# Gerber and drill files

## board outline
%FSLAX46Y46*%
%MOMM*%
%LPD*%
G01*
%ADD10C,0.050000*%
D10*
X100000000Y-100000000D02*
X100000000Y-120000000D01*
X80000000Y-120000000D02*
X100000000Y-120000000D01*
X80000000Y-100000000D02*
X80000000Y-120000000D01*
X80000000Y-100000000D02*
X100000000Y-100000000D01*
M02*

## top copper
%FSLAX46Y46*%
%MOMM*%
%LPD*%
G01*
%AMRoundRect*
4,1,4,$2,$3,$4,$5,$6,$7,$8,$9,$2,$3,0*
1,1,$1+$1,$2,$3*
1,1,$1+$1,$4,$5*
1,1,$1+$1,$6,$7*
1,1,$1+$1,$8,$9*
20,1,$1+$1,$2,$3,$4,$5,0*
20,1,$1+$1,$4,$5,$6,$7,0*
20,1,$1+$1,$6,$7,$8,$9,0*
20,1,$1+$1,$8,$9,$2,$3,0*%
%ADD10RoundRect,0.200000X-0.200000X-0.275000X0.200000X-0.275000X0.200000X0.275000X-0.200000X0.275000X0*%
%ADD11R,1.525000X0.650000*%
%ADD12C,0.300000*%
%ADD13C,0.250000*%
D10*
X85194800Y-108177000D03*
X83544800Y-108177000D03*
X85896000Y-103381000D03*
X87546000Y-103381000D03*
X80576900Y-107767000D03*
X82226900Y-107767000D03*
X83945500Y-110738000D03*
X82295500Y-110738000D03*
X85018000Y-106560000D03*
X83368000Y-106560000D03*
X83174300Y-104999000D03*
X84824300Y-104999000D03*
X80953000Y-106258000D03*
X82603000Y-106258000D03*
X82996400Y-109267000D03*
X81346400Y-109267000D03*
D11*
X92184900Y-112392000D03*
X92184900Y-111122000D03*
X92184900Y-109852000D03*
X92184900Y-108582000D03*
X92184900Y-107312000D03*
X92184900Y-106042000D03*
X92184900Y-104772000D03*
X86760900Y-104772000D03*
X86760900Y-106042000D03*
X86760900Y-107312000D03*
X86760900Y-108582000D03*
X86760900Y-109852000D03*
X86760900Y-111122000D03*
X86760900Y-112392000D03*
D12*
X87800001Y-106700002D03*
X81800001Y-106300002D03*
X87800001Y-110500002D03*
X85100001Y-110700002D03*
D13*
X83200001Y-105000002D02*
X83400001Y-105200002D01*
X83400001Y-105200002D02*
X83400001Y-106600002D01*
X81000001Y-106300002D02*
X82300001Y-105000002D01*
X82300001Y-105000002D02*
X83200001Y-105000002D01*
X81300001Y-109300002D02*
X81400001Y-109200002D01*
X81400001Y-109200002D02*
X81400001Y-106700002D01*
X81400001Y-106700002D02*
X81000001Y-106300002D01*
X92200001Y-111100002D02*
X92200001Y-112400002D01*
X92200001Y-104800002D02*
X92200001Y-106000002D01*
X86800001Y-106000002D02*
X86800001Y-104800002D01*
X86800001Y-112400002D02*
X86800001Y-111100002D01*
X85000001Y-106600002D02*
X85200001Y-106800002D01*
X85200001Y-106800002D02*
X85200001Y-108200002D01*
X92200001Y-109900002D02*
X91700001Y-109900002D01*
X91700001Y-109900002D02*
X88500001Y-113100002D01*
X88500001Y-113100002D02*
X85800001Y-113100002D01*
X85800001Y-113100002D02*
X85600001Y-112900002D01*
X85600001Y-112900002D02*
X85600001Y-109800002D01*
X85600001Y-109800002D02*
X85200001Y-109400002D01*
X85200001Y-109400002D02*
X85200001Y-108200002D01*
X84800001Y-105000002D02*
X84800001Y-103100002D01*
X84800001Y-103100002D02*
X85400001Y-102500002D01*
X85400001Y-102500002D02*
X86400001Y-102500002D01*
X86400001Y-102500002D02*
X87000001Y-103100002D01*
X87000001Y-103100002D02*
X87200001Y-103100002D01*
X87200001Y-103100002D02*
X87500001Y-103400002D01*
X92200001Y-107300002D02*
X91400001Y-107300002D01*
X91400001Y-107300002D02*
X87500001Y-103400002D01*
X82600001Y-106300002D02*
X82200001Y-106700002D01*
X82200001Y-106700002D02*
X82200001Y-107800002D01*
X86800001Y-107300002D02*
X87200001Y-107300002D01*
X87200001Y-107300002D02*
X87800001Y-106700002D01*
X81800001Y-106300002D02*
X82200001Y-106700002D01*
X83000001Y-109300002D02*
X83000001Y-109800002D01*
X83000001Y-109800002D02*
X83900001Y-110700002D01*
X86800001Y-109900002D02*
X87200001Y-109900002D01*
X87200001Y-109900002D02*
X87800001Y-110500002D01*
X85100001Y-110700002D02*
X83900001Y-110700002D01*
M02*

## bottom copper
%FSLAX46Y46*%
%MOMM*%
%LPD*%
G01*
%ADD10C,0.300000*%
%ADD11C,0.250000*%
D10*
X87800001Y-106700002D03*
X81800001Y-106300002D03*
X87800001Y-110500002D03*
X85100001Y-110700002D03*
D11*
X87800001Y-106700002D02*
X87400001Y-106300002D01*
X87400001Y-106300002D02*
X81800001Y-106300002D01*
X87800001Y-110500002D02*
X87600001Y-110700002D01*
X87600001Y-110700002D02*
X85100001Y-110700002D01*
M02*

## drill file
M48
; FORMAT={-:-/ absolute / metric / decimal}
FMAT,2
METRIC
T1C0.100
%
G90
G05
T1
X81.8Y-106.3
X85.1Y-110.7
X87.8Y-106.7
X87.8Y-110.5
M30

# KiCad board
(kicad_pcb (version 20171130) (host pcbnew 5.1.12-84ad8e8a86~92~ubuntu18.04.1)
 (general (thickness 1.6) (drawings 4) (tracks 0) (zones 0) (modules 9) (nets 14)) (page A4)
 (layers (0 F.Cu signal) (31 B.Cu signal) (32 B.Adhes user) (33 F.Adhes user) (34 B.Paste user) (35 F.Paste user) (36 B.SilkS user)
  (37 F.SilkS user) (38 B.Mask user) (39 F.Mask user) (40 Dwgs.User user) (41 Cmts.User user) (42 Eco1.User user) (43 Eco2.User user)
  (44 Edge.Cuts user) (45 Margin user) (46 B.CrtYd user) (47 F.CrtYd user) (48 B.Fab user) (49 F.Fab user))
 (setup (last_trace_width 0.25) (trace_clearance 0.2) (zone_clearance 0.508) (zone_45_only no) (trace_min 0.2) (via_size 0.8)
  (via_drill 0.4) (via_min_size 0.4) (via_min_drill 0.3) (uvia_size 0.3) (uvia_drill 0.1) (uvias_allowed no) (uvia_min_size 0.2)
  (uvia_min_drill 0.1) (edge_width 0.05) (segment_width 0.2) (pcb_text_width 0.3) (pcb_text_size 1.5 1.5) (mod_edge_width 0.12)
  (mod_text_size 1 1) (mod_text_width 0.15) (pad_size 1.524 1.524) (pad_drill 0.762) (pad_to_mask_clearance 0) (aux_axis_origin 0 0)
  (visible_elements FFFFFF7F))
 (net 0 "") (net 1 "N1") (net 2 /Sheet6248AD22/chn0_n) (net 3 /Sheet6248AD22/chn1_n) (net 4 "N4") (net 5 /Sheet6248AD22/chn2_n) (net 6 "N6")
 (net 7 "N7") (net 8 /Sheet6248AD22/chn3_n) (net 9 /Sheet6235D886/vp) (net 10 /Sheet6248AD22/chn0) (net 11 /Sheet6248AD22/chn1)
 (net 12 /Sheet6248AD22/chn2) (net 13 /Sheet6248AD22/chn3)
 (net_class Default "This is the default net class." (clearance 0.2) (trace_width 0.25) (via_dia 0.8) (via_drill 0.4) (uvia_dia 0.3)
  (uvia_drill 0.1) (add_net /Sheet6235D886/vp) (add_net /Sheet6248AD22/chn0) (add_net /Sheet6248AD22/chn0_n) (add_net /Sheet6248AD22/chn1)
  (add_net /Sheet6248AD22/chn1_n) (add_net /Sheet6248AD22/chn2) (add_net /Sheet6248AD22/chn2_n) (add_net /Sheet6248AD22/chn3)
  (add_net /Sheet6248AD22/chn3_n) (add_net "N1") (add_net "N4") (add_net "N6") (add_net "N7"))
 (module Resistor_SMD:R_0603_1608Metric (layer F.Cu) (at 84.369800 108.177000)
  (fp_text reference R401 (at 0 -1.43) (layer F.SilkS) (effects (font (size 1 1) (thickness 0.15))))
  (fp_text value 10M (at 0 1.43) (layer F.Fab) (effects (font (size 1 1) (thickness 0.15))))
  (pad 2 smd roundrect (at 0.825 0) (size 0.8 0.95) (layers F.Cu F.Mask F.Paste) (roundrect_rratio 0.25) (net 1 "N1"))
  (pad 1 smd roundrect (at -0.825 0) (size 0.8 0.95) (layers F.Cu F.Mask F.Paste) (roundrect_rratio 0.25) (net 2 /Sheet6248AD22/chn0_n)))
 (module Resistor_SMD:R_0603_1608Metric (layer F.Cu) (at 86.721000 103.381000)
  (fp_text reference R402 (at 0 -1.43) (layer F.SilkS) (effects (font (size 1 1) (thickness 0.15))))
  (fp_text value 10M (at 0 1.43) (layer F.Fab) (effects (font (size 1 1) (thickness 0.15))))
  (pad 1 smd roundrect (at -0.825 0) (size 0.8 0.95) (layers F.Cu F.Mask F.Paste) (roundrect_rratio 0.25) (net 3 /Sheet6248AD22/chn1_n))
  (pad 2 smd roundrect (at 0.825 0) (size 0.8 0.95) (layers F.Cu F.Mask F.Paste) (roundrect_rratio 0.25) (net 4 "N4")))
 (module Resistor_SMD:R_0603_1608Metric (layer F.Cu) (at 81.401900 107.767000)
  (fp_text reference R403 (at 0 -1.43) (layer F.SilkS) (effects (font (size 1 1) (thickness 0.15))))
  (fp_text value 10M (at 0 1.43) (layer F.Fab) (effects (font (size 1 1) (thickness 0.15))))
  (pad 1 smd roundrect (at -0.825 0) (size 0.8 0.95) (layers F.Cu F.Mask F.Paste) (roundrect_rratio 0.25) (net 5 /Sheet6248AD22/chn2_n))
  (pad 2 smd roundrect (at 0.825 0) (size 0.8 0.95) (layers F.Cu F.Mask F.Paste) (roundrect_rratio 0.25) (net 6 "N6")))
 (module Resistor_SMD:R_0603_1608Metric (layer F.Cu) (at 83.120500 110.738000)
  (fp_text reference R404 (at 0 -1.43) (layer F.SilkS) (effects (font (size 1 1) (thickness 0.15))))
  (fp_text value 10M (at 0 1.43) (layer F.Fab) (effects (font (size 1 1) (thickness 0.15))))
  (pad 2 smd roundrect (at 0.825 0) (size 0.8 0.95) (layers F.Cu F.Mask F.Paste) (roundrect_rratio 0.25) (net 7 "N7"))
  (pad 1 smd roundrect (at -0.825 0) (size 0.8 0.95) (layers F.Cu F.Mask F.Paste) (roundrect_rratio 0.25) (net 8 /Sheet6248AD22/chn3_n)))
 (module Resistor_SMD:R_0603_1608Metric (layer F.Cu) (at 84.193000 106.560000)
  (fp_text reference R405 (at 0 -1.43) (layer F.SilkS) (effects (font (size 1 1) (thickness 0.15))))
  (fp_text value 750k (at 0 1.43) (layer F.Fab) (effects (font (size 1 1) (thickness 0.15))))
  (pad 2 smd roundrect (at 0.825 0) (size 0.8 0.95) (layers F.Cu F.Mask F.Paste) (roundrect_rratio 0.25) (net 1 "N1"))
  (pad 1 smd roundrect (at -0.825 0) (size 0.8 0.95) (layers F.Cu F.Mask F.Paste) (roundrect_rratio 0.25) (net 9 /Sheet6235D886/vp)))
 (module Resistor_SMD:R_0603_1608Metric (layer F.Cu) (at 83.999300 104.999000)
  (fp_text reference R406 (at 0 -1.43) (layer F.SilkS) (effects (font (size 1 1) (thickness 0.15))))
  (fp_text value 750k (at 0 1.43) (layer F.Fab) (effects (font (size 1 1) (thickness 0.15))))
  (pad 1 smd roundrect (at -0.825 0) (size 0.8 0.95) (layers F.Cu F.Mask F.Paste) (roundrect_rratio 0.25) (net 9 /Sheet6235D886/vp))
  (pad 2 smd roundrect (at 0.825 0) (size 0.8 0.95) (layers F.Cu F.Mask F.Paste) (roundrect_rratio 0.25) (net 4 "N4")))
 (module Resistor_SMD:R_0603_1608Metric (layer F.Cu) (at 81.778000 106.258000)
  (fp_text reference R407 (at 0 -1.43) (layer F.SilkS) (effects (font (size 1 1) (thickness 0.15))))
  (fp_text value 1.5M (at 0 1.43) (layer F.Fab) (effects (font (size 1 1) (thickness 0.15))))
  (pad 1 smd roundrect (at -0.825 0) (size 0.8 0.95) (layers F.Cu F.Mask F.Paste) (roundrect_rratio 0.25) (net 9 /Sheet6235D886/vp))
  (pad 2 smd roundrect (at 0.825 0) (size 0.8 0.95) (layers F.Cu F.Mask F.Paste) (roundrect_rratio 0.25) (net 6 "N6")))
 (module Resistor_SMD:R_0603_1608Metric (layer F.Cu) (at 82.171400 109.267000)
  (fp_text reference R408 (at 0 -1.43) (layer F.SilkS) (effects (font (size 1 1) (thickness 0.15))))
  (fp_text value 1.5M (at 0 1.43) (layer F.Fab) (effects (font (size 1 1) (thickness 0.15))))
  (pad 2 smd roundrect (at 0.825 0) (size 0.8 0.95) (layers F.Cu F.Mask F.Paste) (roundrect_rratio 0.25) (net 7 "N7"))
  (pad 1 smd roundrect (at -0.825 0) (size 0.8 0.95) (layers F.Cu F.Mask F.Paste) (roundrect_rratio 0.25) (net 9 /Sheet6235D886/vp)))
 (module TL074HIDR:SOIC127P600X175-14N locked (layer F.Cu) (at 89.472900 108.582000 180.000000)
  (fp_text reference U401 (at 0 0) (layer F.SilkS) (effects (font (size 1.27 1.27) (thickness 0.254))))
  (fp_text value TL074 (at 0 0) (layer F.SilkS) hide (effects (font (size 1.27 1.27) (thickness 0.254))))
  (pad 1 smd rect (at -2.712 -3.81 270.000000) (size 0.65 1.525) (layers F.Cu F.Mask F.Paste) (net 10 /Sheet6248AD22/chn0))
  (pad 2 smd rect (at -2.712 -2.54 270.000000) (size 0.65 1.525) (layers F.Cu F.Mask F.Paste) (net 10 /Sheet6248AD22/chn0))
  (pad 3 smd rect (at -2.712 -1.27 270.000000) (size 0.65 1.525) (layers F.Cu F.Mask F.Paste) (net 1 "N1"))
  (pad 4 smd rect (at -2.712 0 270.000000) (size 0.65 1.525) (layers F.Cu F.Mask F.Paste))
  (pad 5 smd rect (at -2.712 1.27 270.000000) (size 0.65 1.525) (layers F.Cu F.Mask F.Paste) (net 4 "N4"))
  (pad 6 smd rect (at -2.712 2.54 270.000000) (size 0.65 1.525) (layers F.Cu F.Mask F.Paste) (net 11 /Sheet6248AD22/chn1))
  (pad 7 smd rect (at -2.712 3.81 270.000000) (size 0.65 1.525) (layers F.Cu F.Mask F.Paste) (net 11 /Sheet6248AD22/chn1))
  (pad 8 smd rect (at 2.712 3.81 270.000000) (size 0.65 1.525) (layers F.Cu F.Mask F.Paste) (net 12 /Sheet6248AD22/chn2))
  (pad 9 smd rect (at 2.712 2.54 270.000000) (size 0.65 1.525) (layers F.Cu F.Mask F.Paste) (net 12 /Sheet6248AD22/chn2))
  (pad 10 smd rect (at 2.712 1.27 270.000000) (size 0.65 1.525) (layers F.Cu F.Mask F.Paste) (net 6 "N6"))
  (pad 11 smd rect (at 2.712 0 270.000000) (size 0.65 1.525) (layers F.Cu F.Mask F.Paste))
  (pad 12 smd rect (at 2.712 -1.27 270.000000) (size 0.65 1.525) (layers F.Cu F.Mask F.Paste) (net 7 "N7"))
  (pad 13 smd rect (at 2.712 -2.54 270.000000) (size 0.65 1.525) (layers F.Cu F.Mask F.Paste) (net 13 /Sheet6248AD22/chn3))
  (pad 14 smd rect (at 2.712 -3.81 270.000000) (size 0.65 1.525) (layers F.Cu F.Mask F.Paste) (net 13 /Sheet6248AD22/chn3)))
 (gr_line (start 100 100) (end 100 120) (layer Edge.Cuts) (width 0.05))
 (gr_line (start 80 120) (end 100 120) (layer Edge.Cuts) (width 0.05))
 (gr_line (start 80 100) (end 80 120) (layer Edge.Cuts) (width 0.05))
 (gr_line (start 80 100) (end 100 100) (layer Edge.Cuts) (width 0.05))
 (segment (start 83.200001 105.000002) (end 83.400001 105.200002) (width 0.250000) (layer F.Cu) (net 9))
 (segment (start 83.400001 105.200002) (end 83.400001 106.600002) (width 0.250000) (layer F.Cu) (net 9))
 (segment (start 81.000001 106.300002) (end 82.300001 105.000002) (width 0.250000) (layer F.Cu) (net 9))
 (segment (start 82.300001 105.000002) (end 83.200001 105.000002) (width 0.250000) (layer F.Cu) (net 9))
 (segment (start 81.300001 109.300002) (end 81.400001 109.200002) (width 0.250000) (layer F.Cu) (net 9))
 (segment (start 81.400001 109.200002) (end 81.400001 106.700002) (width 0.250000) (layer F.Cu) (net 9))
 (segment (start 81.400001 106.700002) (end 81.000001 106.300002) (width 0.250000) (layer F.Cu) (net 9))
 (segment (start 92.200001 111.100002) (end 92.200001 112.400002) (width 0.250000) (layer F.Cu) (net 10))
 (segment (start 92.200001 104.800002) (end 92.200001 106.000002) (width 0.250000) (layer F.Cu) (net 11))
 (segment (start 86.800001 106.000002) (end 86.800001 104.800002) (width 0.250000) (layer F.Cu) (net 12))
 (segment (start 86.800001 112.400002) (end 86.800001 111.100002) (width 0.250000) (layer F.Cu) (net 13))
 (segment (start 85.000001 106.600002) (end 85.200001 106.800002) (width 0.250000) (layer F.Cu) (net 1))
 (segment (start 85.200001 106.800002) (end 85.200001 108.200002) (width 0.250000) (layer F.Cu) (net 1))
 (segment (start 92.200001 109.900002) (end 91.700001 109.900002) (width 0.250000) (layer F.Cu) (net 1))
 (segment (start 91.700001 109.900002) (end 88.500001 113.100002) (width 0.250000) (layer F.Cu) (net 1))
 (segment (start 88.500001 113.100002) (end 85.800001 113.100002) (width 0.250000) (layer F.Cu) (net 1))
 (segment (start 85.800001 113.100002) (end 85.600001 112.900002) (width 0.250000) (layer F.Cu) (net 1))
 (segment (start 85.600001 112.900002) (end 85.600001 109.800002) (width 0.250000) (layer F.Cu) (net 1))
 (segment (start 85.600001 109.800002) (end 85.200001 109.400002) (width 0.250000) (layer F.Cu) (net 1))
 (segment (start 85.200001 109.400002) (end 85.200001 108.200002) (width 0.250000) (layer F.Cu) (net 1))
 (segment (start 84.800001 105.000002) (end 84.800001 103.100002) (width 0.250000) (layer F.Cu) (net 4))
 (segment (start 84.800001 103.100002) (end 85.400001 102.500002) (width 0.250000) (layer F.Cu) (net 4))
 (segment (start 85.400001 102.500002) (end 86.400001 102.500002) (width 0.250000) (layer F.Cu) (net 4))
 (segment (start 86.400001 102.500002) (end 87.000001 103.100002) (width 0.250000) (layer F.Cu) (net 4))
 (segment (start 87.000001 103.100002) (end 87.200001 103.100002) (width 0.250000) (layer F.Cu) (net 4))
 (segment (start 87.200001 103.100002) (end 87.500001 103.400002) (width 0.250000) (layer F.Cu) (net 4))
 (segment (start 92.200001 107.300002) (end 91.400001 107.300002) (width 0.250000) (layer F.Cu) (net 4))
 (segment (start 91.400001 107.300002) (end 87.500001 103.400002) (width 0.250000) (layer F.Cu) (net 4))
 (segment (start 82.600001 106.300002) (end 82.200001 106.700002) (width 0.250000) (layer F.Cu) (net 6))
 (segment (start 82.200001 106.700002) (end 82.200001 107.800002) (width 0.250000) (layer F.Cu) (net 6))
 (segment (start 86.800001 107.300002) (end 87.200001 107.300002) (width 0.250000) (layer F.Cu) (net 6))
 (segment (start 87.200001 107.300002) (end 87.800001 106.700002) (width 0.250000) (layer F.Cu) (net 6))
 (segment (start 87.800001 106.700002) (end 87.400001 106.300002) (width 0.250000) (layer B.Cu) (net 6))
 (segment (start 87.400001 106.300002) (end 81.800001 106.300002) (width 0.250000) (layer B.Cu) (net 6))
 (segment (start 81.800001 106.300002) (end 82.200001 106.700002) (width 0.250000) (layer F.Cu) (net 6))
 (via micro (at 87.800001 106.700002) (size 0.300000) (drill 0.100000) (layers F.Cu B.Cu) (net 6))
 (via micro (at 81.800001 106.300002) (size 0.300000) (drill 0.100000) (layers F.Cu B.Cu) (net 6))
 (segment (start 83.000001 109.300002) (end 83.000001 109.800002) (width 0.250000) (layer F.Cu) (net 7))
 (segment (start 83.000001 109.800002) (end 83.900001 110.700002) (width 0.250000) (layer F.Cu) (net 7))
 (segment (start 86.800001 109.900002) (end 87.200001 109.900002) (width 0.250000) (layer F.Cu) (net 7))
 (segment (start 87.200001 109.900002) (end 87.800001 110.500002) (width 0.250000) (layer F.Cu) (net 7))
 (segment (start 87.800001 110.500002) (end 87.600001 110.700002) (width 0.250000) (layer B.Cu) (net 7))
 (segment (start 87.600001 110.700002) (end 85.100001 110.700002) (width 0.250000) (layer B.Cu) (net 7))
 (segment (start 85.100001 110.700002) (end 83.900001 110.700002) (width 0.250000) (layer F.Cu) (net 7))
 (via micro (at 87.800001 110.500002) (size 0.300000) (drill 0.100000) (layers F.Cu B.Cu) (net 7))
 (via micro (at 85.100001 110.700002) (size 0.300000) (drill 0.100000) (layers F.Cu B.Cu) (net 7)))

